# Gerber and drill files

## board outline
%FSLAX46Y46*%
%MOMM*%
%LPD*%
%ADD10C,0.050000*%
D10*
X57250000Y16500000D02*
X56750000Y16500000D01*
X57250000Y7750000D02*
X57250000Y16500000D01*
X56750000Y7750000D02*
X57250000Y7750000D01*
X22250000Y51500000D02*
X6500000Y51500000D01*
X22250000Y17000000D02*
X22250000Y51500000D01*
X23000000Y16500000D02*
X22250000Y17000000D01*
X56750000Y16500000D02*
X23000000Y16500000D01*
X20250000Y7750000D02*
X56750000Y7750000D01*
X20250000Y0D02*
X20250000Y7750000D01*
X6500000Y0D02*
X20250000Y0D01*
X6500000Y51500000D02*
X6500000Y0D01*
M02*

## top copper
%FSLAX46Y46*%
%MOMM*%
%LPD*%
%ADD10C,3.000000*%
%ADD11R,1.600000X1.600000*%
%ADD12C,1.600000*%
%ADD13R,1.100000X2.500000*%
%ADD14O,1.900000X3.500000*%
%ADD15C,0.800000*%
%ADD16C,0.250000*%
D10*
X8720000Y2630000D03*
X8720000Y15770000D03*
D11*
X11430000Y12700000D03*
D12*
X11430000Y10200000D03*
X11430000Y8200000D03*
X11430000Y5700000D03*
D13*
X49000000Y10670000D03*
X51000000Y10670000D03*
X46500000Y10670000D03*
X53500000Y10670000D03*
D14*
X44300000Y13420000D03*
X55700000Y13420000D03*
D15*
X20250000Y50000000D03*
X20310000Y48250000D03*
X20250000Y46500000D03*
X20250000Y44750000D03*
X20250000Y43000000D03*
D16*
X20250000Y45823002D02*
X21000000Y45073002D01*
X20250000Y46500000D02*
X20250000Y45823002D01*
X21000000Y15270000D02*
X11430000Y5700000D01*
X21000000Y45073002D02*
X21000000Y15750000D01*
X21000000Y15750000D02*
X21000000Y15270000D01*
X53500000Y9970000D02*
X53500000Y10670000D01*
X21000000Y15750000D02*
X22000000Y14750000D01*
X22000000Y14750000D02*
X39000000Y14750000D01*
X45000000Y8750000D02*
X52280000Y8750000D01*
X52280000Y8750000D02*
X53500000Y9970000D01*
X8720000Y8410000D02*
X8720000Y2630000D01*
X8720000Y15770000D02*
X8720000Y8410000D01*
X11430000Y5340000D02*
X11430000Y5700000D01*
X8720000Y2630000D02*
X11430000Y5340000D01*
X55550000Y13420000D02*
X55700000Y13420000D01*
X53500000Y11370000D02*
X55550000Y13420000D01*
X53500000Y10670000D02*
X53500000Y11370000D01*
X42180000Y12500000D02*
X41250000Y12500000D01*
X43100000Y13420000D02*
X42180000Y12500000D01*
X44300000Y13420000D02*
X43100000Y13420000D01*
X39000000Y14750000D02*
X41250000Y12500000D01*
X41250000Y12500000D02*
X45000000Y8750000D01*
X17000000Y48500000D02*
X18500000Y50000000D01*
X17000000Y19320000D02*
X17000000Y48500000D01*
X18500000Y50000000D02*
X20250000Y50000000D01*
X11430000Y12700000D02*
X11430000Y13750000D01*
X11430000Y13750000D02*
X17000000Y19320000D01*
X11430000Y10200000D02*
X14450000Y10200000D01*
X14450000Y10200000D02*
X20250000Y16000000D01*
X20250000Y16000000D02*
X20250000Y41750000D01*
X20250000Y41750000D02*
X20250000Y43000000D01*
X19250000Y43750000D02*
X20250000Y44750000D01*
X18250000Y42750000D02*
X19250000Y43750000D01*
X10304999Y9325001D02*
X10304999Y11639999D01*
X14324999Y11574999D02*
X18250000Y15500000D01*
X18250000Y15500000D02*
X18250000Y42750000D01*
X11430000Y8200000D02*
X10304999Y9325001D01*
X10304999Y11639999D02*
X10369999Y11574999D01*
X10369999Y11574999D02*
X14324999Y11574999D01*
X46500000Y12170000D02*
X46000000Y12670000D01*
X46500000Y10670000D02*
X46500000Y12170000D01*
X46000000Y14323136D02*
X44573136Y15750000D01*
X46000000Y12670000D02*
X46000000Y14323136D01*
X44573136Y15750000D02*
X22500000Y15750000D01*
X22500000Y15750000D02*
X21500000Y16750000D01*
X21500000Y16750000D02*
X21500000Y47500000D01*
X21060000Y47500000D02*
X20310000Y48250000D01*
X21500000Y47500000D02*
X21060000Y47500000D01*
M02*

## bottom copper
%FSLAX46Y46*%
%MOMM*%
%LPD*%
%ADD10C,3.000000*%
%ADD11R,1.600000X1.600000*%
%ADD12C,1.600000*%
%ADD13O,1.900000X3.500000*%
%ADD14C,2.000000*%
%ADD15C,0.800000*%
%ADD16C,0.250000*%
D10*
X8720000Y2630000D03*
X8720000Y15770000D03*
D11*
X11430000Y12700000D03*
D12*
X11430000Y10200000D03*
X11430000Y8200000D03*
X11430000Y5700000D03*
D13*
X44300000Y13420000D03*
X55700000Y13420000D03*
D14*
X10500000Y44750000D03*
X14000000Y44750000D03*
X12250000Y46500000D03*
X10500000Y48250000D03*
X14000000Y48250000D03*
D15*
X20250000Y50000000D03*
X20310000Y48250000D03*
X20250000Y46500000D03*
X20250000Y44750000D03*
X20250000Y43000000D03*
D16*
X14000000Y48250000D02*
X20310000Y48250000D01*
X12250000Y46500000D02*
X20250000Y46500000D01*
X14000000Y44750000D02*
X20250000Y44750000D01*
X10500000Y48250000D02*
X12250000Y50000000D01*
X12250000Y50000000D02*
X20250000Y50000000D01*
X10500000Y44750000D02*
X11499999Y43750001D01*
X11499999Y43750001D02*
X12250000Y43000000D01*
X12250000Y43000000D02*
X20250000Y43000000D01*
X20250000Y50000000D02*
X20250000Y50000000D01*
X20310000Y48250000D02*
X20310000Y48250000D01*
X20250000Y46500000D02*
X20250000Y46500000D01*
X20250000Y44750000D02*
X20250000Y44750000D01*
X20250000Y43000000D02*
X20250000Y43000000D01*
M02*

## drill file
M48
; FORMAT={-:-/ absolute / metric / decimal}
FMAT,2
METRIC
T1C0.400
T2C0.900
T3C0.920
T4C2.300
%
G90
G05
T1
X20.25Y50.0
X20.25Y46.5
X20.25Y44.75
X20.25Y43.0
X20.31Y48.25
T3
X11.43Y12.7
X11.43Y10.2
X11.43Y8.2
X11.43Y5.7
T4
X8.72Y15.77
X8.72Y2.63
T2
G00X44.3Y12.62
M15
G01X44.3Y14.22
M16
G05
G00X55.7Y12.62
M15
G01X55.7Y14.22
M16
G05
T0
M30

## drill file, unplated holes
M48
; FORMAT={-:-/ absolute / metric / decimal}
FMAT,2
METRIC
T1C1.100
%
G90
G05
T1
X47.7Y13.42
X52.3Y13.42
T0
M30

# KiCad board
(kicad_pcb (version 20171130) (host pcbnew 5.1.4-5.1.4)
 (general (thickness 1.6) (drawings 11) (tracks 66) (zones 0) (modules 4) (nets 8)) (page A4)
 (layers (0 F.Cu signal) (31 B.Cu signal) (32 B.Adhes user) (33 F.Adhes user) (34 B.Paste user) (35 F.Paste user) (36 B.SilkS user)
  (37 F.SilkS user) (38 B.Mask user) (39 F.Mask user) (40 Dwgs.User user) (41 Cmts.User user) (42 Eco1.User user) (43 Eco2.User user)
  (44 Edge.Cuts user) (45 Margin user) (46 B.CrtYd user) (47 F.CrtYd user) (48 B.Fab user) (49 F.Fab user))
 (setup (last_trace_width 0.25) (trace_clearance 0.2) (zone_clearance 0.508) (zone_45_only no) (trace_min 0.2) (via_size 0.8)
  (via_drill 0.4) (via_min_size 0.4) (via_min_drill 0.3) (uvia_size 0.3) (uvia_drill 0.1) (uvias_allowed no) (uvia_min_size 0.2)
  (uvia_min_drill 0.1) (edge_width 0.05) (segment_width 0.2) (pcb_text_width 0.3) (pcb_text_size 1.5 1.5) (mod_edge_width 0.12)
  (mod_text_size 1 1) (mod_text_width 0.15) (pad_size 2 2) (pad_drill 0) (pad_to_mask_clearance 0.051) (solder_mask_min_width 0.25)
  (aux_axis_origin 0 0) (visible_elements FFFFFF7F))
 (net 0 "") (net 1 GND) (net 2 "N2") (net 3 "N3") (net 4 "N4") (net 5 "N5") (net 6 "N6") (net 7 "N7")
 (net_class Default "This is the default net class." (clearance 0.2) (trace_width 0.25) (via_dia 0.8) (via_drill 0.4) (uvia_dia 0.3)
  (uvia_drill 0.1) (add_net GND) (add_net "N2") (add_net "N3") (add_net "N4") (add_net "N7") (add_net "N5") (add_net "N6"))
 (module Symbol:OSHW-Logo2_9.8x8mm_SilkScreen (layer F.Cu) (at 31.5 -12.25)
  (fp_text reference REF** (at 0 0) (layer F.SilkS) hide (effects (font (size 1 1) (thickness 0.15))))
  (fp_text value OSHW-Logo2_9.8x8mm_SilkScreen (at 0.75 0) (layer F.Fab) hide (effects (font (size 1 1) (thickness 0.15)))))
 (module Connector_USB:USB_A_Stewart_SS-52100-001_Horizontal (layer F.Cu) (at 11.43 -12.7 270)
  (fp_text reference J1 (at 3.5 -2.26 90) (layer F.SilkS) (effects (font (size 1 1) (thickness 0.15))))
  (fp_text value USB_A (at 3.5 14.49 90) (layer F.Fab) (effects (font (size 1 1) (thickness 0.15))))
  (pad 5 thru_hole circle (at 10.07 2.71 270) (size 3 3) (drill 2.3) (layers *.Cu *.Mask) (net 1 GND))
  (pad 5 thru_hole circle (at -3.07 2.71 270) (size 3 3) (drill 2.3) (layers *.Cu *.Mask) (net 1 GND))
  (pad 1 thru_hole rect (at 0 0 270) (size 1.6 1.6) (drill 0.92) (layers *.Cu *.Mask) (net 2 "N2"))
  (pad 2 thru_hole circle (at 2.5 0 270) (size 1.6 1.6) (drill 0.92) (layers *.Cu *.Mask) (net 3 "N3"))
  (pad 3 thru_hole circle (at 4.5 0 270) (size 1.6 1.6) (drill 0.92) (layers *.Cu *.Mask) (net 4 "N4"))
  (pad 4 thru_hole circle (at 7 0 270) (size 1.6 1.6) (drill 0.92) (layers *.Cu *.Mask) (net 1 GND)))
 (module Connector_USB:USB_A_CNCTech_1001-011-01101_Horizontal (layer F.Cu) (at 50 -20.32 90)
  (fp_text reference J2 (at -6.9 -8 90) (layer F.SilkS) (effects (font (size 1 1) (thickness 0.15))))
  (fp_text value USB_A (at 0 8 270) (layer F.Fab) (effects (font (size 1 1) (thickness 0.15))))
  (pad 2 smd rect (at -9.65 -1 90) (size 2.5 1.1) (layers F.Cu F.Paste F.Mask) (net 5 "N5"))
  (pad 3 smd rect (at -9.65 1 90) (size 2.5 1.1) (layers F.Cu F.Paste F.Mask) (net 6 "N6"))
  (pad 1 smd rect (at -9.65 -3.5 90) (size 2.5 1.1) (layers F.Cu F.Paste F.Mask) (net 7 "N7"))
  (pad 4 smd rect (at -9.65 3.5 90) (size 2.5 1.1) (layers F.Cu F.Paste F.Mask) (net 1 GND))
  (pad 5 thru_hole oval (at -6.9 -5.7 90) (size 3.5 1.9) (drill oval 2.5 0.9) (layers *.Cu *.Mask) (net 1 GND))
  (pad 5 thru_hole oval (at -6.9 5.7 90) (size 3.5 1.9) (drill oval 2.5 0.9) (layers *.Cu *.Mask) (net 1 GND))
  (pad "" np_thru_hole circle (at -6.9 -2.3 90) (size 1.1 1.1) (drill 1.1) (layers *.Cu *.Mask))
  (pad "" np_thru_hole circle (at -6.9 2.3 90) (size 1.1 1.1) (drill 1.1) (layers *.Cu *.Mask)))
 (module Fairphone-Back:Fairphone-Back (layer F.Cu) (at 12.25 -46.5)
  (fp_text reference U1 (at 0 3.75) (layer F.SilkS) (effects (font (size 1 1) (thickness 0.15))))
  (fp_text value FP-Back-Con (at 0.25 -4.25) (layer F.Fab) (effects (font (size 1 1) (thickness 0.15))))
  (pad d+ connect circle (at -1.75 1.75) (size 2 2) (layers B.Cu B.Mask) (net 3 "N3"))
  (pad d- connect circle (at 1.75 1.75) (size 2 2) (layers B.Cu B.Mask) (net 4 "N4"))
  (pad "" connect circle (at 0 0) (size 2 2) (layers B.Cu B.Mask) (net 1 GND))
  (pad vbus connect circle (at -1.75 -1.75) (size 2 2) (layers B.Cu B.Mask) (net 2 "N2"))
  (pad chrg connect circle (at 1.75 -1.75) (size 2 2) (layers B.Cu B.Mask) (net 7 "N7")))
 (gr_line (start 57.25 -16.5) (end 56.75 -16.5) (layer Edge.Cuts) (width 0.05))
 (gr_line (start 57.25 -7.75) (end 57.25 -16.5) (layer Edge.Cuts) (width 0.05))
 (gr_line (start 56.75 -7.75) (end 57.25 -7.75) (layer Edge.Cuts) (width 0.05))
 (gr_line (start 22.25 -51.5) (end 6.5 -51.5) (layer Edge.Cuts) (width 0.05))
 (gr_line (start 22.25 -17) (end 22.25 -51.5) (layer Edge.Cuts) (width 0.05))
 (gr_line (start 23 -16.5) (end 22.25 -17) (layer Edge.Cuts) (width 0.05))
 (gr_line (start 56.75 -16.5) (end 23 -16.5) (layer Edge.Cuts) (width 0.05))
 (gr_line (start 20.25 -7.75) (end 56.75 -7.75) (layer Edge.Cuts) (width 0.05))
 (gr_line (start 20.25 0) (end 20.25 -7.75) (layer Edge.Cuts) (width 0.05))
 (gr_line (start 6.5 0) (end 20.25 0) (layer Edge.Cuts) (width 0.05))
 (gr_line (start 6.5 -51.5) (end 6.5 0) (layer Edge.Cuts) (width 0.05))
 (segment (start 14 -48.25) (end 20.31 -48.25) (width 0.25) (layer B.Cu) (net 7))
 (segment (start 12.25 -46.5) (end 20.25 -46.5) (width 0.25) (layer B.Cu) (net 1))
 (segment (start 14 -44.75) (end 20.25 -44.75) (width 0.25) (layer B.Cu) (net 4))
 (segment (start 10.5 -48.25) (end 12.25 -50) (width 0.25) (layer B.Cu) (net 2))
 (segment (start 12.25 -50) (end 20.25 -50) (width 0.25) (layer B.Cu) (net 2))
 (segment (start 10.5 -44.75) (end 11.499999 -43.750001) (width 0.25) (layer B.Cu) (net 3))
 (segment (start 11.499999 -43.750001) (end 12.25 -43) (width 0.25) (layer B.Cu) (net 3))
 (segment (start 12.25 -43) (end 20.25 -43) (width 0.25) (layer B.Cu) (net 3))
 (segment (start 20.25 -50) (end 20.25 -50) (width 0.25) (layer B.Cu) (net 2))
 (via (at 20.25 -50) (size 0.8) (drill 0.4) (layers F.Cu B.Cu) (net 2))
 (segment (start 20.31 -48.25) (end 20.31 -48.25) (width 0.25) (layer B.Cu) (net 7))
 (via (at 20.31 -48.25) (size 0.8) (drill 0.4) (layers F.Cu B.Cu) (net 7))
 (segment (start 20.25 -46.5) (end 20.25 -46.5) (width 0.25) (layer B.Cu) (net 1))
 (via (at 20.25 -46.5) (size 0.8) (drill 0.4) (layers F.Cu B.Cu) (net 1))
 (segment (start 20.25 -44.75) (end 20.25 -44.75) (width 0.25) (layer B.Cu) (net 4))
 (via (at 20.25 -44.75) (size 0.8) (drill 0.4) (layers F.Cu B.Cu) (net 4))
 (segment (start 20.25 -43) (end 20.25 -43) (width 0.25) (layer B.Cu) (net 3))
 (via (at 20.25 -43) (size 0.8) (drill 0.4) (layers F.Cu B.Cu) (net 3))
 (segment (start 20.25 -45.823002) (end 21 -45.073002) (width 0.25) (layer F.Cu) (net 1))
 (segment (start 20.25 -46.5) (end 20.25 -45.823002) (width 0.25) (layer F.Cu) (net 1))
 (segment (start 21 -15.27) (end 11.43 -5.7) (width 0.25) (layer F.Cu) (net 1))
 (segment (start 21 -45.073002) (end 21 -15.75) (width 0.25) (layer F.Cu) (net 1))
 (segment (start 21 -15.75) (end 21 -15.27) (width 0.25) (layer F.Cu) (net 1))
 (segment (start 53.5 -9.97) (end 53.5 -10.67) (width 0.25) (layer F.Cu) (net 1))
 (segment (start 21 -15.75) (end 22 -14.75) (width 0.25) (layer F.Cu) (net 1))
 (segment (start 22 -14.75) (end 39 -14.75) (width 0.25) (layer F.Cu) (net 1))
 (segment (start 45 -8.75) (end 52.28 -8.75) (width 0.25) (layer F.Cu) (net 1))
 (segment (start 52.28 -8.75) (end 53.5 -9.97) (width 0.25) (layer F.Cu) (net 1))
 (segment (start 8.72 -8.41) (end 8.72 -2.63) (width 0.25) (layer F.Cu) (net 1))
 (segment (start 8.72 -15.77) (end 8.72 -8.41) (width 0.25) (layer F.Cu) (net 1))
 (segment (start 11.43 -5.34) (end 11.43 -5.7) (width 0.25) (layer F.Cu) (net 1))
 (segment (start 8.72 -2.63) (end 11.43 -5.34) (width 0.25) (layer F.Cu) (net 1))
 (segment (start 55.55 -13.42) (end 55.7 -13.42) (width 0.25) (layer F.Cu) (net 1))
 (segment (start 53.5 -11.37) (end 55.55 -13.42) (width 0.25) (layer F.Cu) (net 1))
 (segment (start 53.5 -10.67) (end 53.5 -11.37) (width 0.25) (layer F.Cu) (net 1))
 (segment (start 42.18 -12.5) (end 41.25 -12.5) (width 0.25) (layer F.Cu) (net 1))
 (segment (start 43.1 -13.42) (end 42.18 -12.5) (width 0.25) (layer F.Cu) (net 1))
 (segment (start 44.3 -13.42) (end 43.1 -13.42) (width 0.25) (layer F.Cu) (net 1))
 (segment (start 39 -14.75) (end 41.25 -12.5) (width 0.25) (layer F.Cu) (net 1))
 (segment (start 41.25 -12.5) (end 45 -8.75) (width 0.25) (layer F.Cu) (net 1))
 (segment (start 17 -48.5) (end 18.5 -50) (width 0.25) (layer F.Cu) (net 2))
 (segment (start 17 -19.32) (end 17 -48.5) (width 0.25) (layer F.Cu) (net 2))
 (segment (start 18.5 -50) (end 20.25 -50) (width 0.25) (layer F.Cu) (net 2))
 (segment (start 11.43 -12.7) (end 11.43 -13.75) (width 0.25) (layer F.Cu) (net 2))
 (segment (start 11.43 -13.75) (end 17 -19.32) (width 0.25) (layer F.Cu) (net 2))
 (segment (start 11.43 -10.2) (end 14.45 -10.2) (width 0.25) (layer F.Cu) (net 3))
 (segment (start 14.45 -10.2) (end 20.25 -16) (width 0.25) (layer F.Cu) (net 3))
 (segment (start 20.25 -16) (end 20.25 -41.75) (width 0.25) (layer F.Cu) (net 3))
 (segment (start 20.25 -41.75) (end 20.25 -43) (width 0.25) (layer F.Cu) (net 3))
 (segment (start 19.25 -43.75) (end 20.25 -44.75) (width 0.25) (layer F.Cu) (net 4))
 (segment (start 18.25 -42.75) (end 19.25 -43.75) (width 0.25) (layer F.Cu) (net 4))
 (segment (start 10.304999 -9.325001) (end 10.304999 -11.639999) (width 0.25) (layer F.Cu) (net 4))
 (segment (start 14.324999 -11.574999) (end 18.25 -15.5) (width 0.25) (layer F.Cu) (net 4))
 (segment (start 18.25 -15.5) (end 18.25 -42.75) (width 0.25) (layer F.Cu) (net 4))
 (segment (start 11.43 -8.2) (end 10.304999 -9.325001) (width 0.25) (layer F.Cu) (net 4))
 (segment (start 10.304999 -11.639999) (end 10.369999 -11.574999) (width 0.25) (layer F.Cu) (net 4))
 (segment (start 10.369999 -11.574999) (end 14.324999 -11.574999) (width 0.25) (layer F.Cu) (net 4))
 (segment (start 46.5 -12.17) (end 46 -12.67) (width 0.25) (layer F.Cu) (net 7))
 (segment (start 46.5 -10.67) (end 46.5 -12.17) (width 0.25) (layer F.Cu) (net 7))
 (segment (start 46 -14.323136) (end 44.573136 -15.75) (width 0.25) (layer F.Cu) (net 7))
 (segment (start 46 -12.67) (end 46 -14.323136) (width 0.25) (layer F.Cu) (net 7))
 (segment (start 44.573136 -15.75) (end 22.5 -15.75) (width 0.25) (layer F.Cu) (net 7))
 (segment (start 22.5 -15.75) (end 21.5 -16.75) (width 0.25) (layer F.Cu) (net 7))
 (segment (start 21.5 -16.75) (end 21.5 -47.5) (width 0.25) (layer F.Cu) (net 7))
 (segment (start 21.06 -47.5) (end 20.31 -48.25) (width 0.25) (layer F.Cu) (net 7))
 (segment (start 21.5 -47.5) (end 21.06 -47.5) (width 0.25) (layer F.Cu) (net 7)))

